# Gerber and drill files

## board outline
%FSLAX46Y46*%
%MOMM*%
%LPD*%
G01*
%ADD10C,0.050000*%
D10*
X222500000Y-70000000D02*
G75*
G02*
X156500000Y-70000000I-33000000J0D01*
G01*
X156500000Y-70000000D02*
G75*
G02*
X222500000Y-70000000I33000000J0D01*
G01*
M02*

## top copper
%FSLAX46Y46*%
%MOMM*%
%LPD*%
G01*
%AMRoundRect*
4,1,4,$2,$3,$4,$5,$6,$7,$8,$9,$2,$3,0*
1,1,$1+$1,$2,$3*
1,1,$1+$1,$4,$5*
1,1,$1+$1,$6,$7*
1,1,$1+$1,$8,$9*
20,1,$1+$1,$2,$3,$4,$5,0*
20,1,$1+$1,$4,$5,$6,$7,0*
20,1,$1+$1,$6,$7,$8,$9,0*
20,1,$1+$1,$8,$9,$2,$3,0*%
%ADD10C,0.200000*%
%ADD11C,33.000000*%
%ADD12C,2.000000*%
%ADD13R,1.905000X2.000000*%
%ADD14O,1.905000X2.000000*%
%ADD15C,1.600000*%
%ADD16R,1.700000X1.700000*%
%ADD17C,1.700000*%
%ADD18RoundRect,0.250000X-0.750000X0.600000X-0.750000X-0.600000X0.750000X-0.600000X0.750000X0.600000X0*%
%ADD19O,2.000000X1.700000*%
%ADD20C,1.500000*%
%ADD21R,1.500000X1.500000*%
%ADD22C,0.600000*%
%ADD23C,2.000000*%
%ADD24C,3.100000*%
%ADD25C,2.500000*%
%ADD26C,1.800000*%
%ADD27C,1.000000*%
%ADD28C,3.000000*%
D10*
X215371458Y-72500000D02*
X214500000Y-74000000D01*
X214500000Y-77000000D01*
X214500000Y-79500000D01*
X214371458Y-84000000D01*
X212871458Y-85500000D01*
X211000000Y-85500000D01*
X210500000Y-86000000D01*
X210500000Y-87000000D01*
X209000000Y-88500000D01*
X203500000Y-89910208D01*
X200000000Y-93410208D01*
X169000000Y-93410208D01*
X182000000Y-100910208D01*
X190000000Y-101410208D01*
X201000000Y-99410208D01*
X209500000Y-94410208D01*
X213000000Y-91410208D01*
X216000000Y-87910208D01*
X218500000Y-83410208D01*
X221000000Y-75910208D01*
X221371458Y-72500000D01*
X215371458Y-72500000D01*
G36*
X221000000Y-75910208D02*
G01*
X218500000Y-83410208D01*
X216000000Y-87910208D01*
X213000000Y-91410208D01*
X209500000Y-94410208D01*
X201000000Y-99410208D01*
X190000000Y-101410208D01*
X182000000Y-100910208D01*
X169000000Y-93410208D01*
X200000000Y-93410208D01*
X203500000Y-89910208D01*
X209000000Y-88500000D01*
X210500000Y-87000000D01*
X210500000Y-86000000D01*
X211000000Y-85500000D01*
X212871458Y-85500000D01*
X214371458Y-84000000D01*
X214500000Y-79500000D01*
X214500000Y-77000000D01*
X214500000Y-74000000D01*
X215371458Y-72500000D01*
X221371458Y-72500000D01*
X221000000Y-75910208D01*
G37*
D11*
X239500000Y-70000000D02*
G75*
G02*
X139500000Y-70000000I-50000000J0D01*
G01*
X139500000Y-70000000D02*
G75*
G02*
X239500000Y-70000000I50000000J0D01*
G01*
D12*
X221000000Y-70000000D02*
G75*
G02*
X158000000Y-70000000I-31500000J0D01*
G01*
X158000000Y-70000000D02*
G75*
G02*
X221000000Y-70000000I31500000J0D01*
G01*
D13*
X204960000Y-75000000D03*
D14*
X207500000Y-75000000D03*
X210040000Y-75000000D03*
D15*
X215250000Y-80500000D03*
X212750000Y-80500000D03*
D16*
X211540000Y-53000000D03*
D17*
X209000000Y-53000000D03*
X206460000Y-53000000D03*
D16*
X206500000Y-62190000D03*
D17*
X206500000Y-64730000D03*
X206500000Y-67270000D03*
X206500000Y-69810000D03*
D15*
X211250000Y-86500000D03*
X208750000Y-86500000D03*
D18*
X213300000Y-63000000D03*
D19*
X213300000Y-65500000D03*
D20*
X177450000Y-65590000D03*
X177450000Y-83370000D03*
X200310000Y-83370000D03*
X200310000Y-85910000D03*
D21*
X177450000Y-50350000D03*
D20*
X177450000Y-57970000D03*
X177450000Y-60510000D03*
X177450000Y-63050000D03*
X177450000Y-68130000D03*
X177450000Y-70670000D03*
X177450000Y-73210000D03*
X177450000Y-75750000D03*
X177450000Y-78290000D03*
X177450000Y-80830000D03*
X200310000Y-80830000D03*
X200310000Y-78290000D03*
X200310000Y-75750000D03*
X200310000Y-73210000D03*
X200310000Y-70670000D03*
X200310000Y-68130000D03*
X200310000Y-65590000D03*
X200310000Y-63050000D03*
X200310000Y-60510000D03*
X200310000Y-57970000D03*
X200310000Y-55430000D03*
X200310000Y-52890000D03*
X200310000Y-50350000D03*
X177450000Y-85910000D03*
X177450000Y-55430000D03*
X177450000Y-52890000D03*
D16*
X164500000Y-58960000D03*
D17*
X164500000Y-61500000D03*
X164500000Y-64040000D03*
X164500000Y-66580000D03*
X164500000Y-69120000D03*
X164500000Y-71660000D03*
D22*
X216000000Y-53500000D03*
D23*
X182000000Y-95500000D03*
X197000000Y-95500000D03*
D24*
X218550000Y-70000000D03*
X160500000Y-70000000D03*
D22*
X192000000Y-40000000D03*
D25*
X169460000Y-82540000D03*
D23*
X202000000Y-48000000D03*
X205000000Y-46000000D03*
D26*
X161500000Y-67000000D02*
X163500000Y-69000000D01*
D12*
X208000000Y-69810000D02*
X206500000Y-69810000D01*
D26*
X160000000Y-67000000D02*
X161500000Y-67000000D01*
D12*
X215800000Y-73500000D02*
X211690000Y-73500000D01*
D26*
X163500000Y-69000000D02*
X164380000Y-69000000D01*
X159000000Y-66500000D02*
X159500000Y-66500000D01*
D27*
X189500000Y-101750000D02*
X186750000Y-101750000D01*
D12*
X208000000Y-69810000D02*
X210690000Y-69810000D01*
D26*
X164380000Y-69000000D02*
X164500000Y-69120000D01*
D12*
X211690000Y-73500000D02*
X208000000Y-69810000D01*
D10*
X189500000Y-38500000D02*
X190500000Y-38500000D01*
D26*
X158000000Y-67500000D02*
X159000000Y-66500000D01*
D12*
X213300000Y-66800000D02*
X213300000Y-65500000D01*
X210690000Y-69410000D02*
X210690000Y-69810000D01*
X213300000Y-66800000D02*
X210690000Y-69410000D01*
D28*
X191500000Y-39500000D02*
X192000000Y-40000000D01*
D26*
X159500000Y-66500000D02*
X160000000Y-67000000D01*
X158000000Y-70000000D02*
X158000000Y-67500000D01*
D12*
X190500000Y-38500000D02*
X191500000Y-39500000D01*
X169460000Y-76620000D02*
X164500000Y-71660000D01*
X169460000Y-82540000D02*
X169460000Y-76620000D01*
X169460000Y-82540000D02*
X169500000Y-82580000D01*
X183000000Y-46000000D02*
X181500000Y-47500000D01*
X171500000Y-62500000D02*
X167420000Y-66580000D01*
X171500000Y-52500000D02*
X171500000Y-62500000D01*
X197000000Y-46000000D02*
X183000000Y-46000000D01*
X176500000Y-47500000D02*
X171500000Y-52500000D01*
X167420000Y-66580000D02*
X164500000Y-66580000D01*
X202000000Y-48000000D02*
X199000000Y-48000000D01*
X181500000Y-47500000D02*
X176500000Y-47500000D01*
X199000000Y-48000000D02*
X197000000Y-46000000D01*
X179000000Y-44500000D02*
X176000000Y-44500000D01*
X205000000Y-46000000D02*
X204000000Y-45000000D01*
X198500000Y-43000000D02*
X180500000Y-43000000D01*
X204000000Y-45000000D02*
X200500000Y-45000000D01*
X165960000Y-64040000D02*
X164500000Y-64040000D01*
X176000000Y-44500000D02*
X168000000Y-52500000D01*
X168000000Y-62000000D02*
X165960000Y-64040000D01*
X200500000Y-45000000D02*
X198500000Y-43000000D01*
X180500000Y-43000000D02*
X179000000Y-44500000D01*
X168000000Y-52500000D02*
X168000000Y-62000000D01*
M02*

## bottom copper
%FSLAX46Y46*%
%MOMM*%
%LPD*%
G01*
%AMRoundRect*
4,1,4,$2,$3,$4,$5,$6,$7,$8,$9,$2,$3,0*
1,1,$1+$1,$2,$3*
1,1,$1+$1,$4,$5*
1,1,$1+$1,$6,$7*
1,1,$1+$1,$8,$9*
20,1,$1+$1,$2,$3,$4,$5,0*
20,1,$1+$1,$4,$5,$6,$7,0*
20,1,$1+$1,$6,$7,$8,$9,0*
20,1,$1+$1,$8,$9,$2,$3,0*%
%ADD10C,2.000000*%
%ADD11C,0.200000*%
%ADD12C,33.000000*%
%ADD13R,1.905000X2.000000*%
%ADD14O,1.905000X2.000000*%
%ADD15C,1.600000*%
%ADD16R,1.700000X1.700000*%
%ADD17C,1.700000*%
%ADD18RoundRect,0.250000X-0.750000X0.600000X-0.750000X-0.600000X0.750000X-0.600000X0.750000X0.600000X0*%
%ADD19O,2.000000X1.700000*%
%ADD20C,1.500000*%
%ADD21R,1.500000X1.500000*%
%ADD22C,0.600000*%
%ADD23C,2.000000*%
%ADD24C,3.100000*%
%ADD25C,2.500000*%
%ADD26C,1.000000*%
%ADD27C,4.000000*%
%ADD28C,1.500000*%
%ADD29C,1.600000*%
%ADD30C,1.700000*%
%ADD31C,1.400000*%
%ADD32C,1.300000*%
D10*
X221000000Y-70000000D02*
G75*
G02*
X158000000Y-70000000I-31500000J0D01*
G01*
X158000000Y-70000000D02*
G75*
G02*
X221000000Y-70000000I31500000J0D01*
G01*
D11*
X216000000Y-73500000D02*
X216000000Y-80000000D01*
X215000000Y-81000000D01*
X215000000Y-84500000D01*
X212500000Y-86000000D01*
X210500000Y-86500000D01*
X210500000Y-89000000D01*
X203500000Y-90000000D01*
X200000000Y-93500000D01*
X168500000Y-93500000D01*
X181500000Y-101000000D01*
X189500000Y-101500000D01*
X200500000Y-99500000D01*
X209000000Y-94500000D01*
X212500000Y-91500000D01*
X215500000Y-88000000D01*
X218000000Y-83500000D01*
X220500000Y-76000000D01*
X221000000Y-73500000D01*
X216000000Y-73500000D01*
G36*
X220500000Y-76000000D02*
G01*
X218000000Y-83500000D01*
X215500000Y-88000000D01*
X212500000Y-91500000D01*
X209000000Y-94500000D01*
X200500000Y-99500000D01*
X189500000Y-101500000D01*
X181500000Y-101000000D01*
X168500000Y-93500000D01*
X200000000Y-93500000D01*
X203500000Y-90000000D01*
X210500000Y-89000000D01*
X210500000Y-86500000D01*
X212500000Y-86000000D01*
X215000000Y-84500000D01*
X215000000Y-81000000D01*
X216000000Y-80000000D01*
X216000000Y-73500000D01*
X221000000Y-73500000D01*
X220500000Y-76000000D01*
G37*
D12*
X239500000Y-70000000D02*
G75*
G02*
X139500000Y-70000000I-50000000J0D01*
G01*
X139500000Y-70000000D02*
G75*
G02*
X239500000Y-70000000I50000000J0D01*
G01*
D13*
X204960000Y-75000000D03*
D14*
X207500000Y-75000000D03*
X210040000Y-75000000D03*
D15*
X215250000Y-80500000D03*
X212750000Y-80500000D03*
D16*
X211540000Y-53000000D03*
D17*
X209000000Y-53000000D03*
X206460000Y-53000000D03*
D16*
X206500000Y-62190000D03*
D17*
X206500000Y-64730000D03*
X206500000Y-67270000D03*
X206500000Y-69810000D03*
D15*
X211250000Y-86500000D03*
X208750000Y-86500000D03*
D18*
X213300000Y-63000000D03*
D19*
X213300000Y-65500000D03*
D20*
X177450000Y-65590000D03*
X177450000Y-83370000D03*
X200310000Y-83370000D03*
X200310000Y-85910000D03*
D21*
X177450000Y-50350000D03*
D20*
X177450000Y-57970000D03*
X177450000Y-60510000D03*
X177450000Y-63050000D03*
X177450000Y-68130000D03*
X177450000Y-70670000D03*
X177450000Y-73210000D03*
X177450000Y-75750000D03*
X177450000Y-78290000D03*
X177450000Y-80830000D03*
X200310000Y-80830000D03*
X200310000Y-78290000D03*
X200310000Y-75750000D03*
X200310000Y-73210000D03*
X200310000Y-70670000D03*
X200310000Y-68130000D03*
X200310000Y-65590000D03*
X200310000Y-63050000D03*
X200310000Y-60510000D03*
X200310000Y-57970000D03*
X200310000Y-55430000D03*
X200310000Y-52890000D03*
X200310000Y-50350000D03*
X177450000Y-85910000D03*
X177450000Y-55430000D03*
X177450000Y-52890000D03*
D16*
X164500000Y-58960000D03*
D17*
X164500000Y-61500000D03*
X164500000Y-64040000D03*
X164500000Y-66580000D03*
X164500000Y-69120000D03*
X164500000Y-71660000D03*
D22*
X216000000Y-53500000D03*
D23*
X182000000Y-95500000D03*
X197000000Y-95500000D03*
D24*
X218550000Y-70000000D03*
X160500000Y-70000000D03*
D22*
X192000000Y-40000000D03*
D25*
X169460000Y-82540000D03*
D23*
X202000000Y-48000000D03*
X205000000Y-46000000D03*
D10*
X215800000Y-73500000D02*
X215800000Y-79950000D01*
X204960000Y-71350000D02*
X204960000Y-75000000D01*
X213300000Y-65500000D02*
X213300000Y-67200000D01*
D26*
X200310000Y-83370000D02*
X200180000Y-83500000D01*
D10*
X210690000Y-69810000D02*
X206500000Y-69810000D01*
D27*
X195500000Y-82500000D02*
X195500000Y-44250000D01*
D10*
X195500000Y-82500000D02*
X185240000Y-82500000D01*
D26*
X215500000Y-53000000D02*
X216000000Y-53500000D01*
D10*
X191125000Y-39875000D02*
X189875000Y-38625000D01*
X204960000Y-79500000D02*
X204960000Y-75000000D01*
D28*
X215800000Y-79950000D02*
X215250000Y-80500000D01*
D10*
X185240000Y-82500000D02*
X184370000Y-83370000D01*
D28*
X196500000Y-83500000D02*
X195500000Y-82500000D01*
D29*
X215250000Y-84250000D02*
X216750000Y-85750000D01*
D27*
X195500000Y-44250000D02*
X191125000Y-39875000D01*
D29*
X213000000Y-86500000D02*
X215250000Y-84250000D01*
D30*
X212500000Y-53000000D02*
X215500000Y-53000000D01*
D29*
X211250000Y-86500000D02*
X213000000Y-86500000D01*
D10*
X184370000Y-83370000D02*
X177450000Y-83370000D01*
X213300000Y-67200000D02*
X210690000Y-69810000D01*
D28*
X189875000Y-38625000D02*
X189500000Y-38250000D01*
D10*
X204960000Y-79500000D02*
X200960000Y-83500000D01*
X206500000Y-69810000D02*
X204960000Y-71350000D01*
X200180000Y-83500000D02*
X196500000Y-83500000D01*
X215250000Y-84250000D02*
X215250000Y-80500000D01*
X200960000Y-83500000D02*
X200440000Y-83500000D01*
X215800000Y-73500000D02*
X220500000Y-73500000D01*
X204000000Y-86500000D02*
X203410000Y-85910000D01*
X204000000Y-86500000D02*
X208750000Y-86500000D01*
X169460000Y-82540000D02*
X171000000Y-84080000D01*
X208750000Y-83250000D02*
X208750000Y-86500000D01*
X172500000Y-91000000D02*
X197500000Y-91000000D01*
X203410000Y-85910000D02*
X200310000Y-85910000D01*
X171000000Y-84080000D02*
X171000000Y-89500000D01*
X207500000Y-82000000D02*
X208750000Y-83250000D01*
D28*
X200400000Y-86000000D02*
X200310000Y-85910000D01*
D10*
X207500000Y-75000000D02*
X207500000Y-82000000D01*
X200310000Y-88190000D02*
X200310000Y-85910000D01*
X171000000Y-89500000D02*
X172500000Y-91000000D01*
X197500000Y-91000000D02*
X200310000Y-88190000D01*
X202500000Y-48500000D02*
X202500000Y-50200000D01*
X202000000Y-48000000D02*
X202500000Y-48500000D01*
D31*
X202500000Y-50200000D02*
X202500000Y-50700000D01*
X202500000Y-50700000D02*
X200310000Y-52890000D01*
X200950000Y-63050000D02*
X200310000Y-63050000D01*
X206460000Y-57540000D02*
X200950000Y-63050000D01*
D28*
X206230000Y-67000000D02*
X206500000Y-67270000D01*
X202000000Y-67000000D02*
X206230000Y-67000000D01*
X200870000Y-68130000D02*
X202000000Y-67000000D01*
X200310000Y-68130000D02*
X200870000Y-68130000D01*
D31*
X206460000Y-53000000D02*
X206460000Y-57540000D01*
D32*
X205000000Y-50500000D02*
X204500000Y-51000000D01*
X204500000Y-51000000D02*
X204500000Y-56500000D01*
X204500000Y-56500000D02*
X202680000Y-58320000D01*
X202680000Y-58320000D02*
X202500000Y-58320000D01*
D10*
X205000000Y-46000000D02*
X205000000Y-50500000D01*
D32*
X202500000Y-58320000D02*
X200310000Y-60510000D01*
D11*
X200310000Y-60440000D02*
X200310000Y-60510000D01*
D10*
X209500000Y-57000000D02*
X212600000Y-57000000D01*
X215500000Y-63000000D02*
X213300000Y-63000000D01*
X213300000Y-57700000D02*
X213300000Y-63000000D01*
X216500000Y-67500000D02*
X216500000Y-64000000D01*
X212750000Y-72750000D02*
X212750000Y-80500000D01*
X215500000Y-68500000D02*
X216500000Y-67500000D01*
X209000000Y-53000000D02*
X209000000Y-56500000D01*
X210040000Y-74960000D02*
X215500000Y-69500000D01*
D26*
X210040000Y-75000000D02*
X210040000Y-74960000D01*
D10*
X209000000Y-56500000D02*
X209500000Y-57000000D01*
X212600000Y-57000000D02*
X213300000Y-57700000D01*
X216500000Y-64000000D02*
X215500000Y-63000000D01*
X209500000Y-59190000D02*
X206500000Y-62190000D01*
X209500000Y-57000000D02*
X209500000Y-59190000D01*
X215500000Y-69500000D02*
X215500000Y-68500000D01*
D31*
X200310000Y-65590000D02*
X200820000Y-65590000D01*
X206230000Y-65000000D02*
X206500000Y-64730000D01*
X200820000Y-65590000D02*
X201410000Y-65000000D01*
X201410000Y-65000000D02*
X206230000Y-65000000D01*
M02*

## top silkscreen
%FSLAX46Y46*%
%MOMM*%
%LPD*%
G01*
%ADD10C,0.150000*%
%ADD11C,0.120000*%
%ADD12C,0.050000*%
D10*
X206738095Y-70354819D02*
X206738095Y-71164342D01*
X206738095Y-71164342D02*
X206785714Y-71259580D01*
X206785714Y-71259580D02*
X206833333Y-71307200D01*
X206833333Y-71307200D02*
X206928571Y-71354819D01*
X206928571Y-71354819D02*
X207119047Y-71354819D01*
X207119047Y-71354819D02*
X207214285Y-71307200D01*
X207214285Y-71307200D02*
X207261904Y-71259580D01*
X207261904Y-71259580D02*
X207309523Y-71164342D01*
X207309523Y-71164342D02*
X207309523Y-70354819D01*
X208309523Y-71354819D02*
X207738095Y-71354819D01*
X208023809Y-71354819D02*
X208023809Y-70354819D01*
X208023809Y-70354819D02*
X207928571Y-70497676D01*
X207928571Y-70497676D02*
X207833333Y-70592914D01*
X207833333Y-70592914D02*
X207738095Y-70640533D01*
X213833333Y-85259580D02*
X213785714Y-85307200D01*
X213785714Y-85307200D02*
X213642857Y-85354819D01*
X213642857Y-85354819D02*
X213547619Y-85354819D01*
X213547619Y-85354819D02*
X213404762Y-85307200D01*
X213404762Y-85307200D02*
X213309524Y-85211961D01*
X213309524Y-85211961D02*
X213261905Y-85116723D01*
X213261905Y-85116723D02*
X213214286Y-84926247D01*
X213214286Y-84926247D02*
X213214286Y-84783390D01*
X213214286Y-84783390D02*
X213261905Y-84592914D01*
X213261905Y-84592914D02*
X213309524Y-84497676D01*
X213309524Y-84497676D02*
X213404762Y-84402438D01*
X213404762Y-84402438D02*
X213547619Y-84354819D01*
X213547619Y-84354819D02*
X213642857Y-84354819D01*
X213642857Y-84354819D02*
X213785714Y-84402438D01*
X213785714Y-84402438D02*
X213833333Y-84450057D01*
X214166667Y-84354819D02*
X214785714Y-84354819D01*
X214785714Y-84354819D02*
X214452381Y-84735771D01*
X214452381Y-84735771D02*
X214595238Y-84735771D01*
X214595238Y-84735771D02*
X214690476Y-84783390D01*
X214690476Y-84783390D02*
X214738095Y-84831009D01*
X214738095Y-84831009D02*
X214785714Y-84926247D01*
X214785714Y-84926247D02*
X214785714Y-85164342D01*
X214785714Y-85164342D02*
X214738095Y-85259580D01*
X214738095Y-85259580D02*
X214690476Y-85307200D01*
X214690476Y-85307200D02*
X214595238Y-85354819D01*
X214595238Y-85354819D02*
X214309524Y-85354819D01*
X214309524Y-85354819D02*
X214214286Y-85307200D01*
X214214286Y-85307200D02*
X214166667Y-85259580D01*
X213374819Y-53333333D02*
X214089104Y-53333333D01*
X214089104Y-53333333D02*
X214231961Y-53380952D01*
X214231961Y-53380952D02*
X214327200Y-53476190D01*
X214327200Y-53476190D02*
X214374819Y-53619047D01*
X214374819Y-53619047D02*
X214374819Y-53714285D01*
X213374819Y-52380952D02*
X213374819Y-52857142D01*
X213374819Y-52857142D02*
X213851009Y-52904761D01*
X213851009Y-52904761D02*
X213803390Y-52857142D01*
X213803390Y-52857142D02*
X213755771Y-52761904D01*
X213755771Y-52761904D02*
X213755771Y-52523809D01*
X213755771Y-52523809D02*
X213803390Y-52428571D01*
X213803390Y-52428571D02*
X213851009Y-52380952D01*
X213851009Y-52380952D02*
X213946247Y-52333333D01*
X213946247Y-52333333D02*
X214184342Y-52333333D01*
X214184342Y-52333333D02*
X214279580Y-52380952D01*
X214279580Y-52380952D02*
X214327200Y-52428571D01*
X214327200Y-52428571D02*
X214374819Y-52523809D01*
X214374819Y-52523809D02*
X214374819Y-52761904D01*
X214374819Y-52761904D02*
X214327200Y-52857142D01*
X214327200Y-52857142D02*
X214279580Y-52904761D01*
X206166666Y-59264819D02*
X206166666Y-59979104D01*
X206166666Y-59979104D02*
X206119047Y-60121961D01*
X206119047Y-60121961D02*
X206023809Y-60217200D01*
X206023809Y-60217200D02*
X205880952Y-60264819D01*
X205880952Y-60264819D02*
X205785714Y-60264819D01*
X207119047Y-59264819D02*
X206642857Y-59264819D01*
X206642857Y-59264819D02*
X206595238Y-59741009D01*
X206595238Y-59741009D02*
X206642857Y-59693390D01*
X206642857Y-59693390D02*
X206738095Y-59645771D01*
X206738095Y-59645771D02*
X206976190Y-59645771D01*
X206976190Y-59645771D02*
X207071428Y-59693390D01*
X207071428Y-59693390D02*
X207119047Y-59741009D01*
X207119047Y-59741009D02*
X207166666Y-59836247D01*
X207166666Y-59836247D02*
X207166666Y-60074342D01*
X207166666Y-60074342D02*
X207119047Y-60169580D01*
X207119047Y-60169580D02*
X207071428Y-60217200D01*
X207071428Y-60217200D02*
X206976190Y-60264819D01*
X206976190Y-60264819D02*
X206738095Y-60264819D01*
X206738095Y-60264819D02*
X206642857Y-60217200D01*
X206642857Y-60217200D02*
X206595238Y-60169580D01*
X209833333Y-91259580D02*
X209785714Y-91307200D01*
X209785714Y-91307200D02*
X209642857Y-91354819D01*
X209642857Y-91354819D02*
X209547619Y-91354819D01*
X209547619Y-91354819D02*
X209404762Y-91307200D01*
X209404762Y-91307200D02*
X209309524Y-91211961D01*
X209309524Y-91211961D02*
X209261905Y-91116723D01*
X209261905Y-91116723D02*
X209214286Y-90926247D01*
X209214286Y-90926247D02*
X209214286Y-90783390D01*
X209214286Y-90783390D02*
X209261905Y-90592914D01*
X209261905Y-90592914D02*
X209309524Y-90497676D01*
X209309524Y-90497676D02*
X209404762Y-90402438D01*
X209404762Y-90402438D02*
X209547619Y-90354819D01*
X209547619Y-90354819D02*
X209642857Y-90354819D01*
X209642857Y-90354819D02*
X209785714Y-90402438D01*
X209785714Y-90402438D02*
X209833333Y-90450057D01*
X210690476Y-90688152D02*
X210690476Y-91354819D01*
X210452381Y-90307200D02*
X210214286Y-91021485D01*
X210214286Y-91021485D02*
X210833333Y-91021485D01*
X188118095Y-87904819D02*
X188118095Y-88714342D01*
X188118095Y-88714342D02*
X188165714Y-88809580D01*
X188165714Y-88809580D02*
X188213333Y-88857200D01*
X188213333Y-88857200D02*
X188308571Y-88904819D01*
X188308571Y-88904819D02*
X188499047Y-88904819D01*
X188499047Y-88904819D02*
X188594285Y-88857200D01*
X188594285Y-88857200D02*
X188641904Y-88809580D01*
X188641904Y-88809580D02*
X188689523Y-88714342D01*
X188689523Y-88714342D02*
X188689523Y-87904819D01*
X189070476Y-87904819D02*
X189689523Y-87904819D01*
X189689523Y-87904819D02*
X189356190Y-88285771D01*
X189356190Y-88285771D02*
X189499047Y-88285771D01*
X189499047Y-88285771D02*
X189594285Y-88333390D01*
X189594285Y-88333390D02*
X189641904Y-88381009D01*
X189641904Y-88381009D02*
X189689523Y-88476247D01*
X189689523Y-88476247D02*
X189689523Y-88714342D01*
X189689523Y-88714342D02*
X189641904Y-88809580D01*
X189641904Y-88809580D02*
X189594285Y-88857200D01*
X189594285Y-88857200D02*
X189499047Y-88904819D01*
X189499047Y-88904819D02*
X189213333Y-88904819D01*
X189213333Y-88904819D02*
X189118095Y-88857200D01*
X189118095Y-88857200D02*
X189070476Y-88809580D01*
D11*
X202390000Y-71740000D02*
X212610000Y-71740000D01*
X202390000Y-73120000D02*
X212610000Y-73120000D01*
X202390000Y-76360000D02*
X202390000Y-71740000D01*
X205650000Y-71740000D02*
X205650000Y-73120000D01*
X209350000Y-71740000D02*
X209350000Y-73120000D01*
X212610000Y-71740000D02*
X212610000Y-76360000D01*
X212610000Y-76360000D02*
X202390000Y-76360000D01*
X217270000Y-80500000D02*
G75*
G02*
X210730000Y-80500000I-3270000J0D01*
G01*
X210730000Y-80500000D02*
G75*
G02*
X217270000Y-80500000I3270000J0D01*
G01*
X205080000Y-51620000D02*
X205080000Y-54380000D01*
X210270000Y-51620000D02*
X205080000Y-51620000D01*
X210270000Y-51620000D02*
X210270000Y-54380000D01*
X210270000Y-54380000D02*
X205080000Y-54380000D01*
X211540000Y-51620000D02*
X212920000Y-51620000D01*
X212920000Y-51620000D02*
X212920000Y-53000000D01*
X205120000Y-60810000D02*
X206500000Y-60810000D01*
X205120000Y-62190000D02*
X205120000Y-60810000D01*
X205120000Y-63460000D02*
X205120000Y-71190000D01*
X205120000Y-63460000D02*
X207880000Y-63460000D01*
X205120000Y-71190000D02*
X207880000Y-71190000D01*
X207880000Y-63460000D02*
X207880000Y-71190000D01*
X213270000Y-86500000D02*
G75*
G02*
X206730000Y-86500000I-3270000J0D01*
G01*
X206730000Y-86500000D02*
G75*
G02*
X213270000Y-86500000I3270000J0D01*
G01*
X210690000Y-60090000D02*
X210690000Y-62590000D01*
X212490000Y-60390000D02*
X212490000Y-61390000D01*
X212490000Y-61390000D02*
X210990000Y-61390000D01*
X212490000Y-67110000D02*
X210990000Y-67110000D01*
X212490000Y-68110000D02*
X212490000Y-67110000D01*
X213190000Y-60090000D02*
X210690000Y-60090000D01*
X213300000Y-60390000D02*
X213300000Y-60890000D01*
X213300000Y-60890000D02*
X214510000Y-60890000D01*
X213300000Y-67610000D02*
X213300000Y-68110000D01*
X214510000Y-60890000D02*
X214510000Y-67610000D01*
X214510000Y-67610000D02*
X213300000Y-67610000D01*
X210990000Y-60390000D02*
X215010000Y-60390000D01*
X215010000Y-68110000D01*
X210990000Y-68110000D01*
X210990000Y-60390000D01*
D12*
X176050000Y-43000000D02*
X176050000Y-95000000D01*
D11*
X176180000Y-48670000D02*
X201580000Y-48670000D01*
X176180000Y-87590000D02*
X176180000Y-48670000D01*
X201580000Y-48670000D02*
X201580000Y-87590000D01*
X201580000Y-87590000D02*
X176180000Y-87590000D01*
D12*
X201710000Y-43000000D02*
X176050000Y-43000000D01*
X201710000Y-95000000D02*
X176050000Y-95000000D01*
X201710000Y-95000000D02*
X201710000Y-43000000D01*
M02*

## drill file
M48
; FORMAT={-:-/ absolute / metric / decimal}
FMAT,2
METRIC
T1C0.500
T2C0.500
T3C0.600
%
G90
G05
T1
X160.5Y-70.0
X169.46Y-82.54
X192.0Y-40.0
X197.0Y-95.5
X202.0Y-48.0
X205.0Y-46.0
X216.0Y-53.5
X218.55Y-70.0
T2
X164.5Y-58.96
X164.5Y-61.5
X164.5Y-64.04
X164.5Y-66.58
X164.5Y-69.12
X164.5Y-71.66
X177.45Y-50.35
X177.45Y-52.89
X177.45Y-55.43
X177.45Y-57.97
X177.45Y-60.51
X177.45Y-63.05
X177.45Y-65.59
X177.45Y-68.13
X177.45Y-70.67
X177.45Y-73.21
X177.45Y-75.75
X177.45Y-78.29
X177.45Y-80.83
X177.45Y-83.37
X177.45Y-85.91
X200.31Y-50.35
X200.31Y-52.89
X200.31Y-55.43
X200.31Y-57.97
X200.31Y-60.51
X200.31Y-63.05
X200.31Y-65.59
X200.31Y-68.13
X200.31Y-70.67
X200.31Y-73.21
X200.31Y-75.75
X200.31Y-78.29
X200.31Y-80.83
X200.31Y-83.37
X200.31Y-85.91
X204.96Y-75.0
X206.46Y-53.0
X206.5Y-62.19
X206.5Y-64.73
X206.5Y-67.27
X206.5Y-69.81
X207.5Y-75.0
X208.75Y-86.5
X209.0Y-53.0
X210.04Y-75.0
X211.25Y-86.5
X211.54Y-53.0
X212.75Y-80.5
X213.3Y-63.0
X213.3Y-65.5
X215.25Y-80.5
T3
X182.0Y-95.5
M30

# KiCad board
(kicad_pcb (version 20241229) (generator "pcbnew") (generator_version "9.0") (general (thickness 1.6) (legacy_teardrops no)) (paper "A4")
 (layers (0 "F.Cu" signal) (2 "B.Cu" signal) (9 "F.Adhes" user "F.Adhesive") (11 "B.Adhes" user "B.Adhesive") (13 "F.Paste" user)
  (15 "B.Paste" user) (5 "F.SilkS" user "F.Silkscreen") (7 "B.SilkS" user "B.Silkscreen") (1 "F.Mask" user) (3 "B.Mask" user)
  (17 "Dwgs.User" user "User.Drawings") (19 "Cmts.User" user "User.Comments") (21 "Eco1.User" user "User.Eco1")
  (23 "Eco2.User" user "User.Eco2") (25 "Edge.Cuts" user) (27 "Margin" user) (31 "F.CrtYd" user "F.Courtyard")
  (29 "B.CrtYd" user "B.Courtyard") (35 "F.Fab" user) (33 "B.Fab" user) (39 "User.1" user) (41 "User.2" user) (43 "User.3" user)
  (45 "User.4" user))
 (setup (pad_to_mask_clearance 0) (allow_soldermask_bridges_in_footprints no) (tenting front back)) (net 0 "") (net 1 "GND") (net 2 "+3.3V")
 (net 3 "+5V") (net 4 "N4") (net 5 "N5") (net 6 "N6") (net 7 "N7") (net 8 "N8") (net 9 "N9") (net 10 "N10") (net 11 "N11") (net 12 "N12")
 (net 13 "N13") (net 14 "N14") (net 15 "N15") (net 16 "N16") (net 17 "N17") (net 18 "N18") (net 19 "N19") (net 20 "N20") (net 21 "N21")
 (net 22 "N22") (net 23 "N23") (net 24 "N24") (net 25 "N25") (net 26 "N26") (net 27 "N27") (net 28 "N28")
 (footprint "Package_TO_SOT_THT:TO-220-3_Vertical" (layer "F.Cu") (at 204.96 75)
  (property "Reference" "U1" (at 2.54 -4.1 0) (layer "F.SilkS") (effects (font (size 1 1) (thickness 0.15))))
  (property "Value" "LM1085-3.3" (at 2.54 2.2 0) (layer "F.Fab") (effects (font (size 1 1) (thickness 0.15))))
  (fp_line (start -2.57 -3.26) (end 7.65 -3.26) (stroke (width 0.12) (type solid)) (layer "F.SilkS"))
  (fp_line (start -2.57 -1.88) (end 7.65 -1.88) (stroke (width 0.12) (type solid)) (layer "F.SilkS"))
  (fp_line (start -2.57 1.36) (end -2.57 -3.26) (stroke (width 0.12) (type solid)) (layer "F.SilkS"))
  (fp_line (start 0.69 -3.26) (end 0.69 -1.88) (stroke (width 0.12) (type solid)) (layer "F.SilkS"))
  (fp_line (start 4.39 -3.26) (end 4.39 -1.88) (stroke (width 0.12) (type solid)) (layer "F.SilkS"))
  (fp_line (start 7.65 -3.26) (end 7.65 1.36) (stroke (width 0.12) (type solid)) (layer "F.SilkS"))
  (fp_line (start 7.65 1.36) (end -2.57 1.36) (stroke (width 0.12) (type solid)) (layer "F.SilkS"))
  (pad "1" thru_hole rect (at 0 0) (size 1.905 2) (drill 0.5) (layers "*.Cu" "*.Mask") (remove_unused_layers no) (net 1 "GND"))
  (pad "2" thru_hole oval (at 2.54 0) (size 1.905 2) (drill 0.5) (layers "*.Cu" "*.Mask") (remove_unused_layers no) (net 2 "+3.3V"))
  (pad "3" thru_hole oval (at 5.08 0) (size 1.905 2) (drill 0.5) (layers "*.Cu" "*.Mask") (remove_unused_layers no) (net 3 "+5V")))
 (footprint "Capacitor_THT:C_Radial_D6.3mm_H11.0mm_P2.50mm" (layer "F.Cu") (at 215.25 80.5 180)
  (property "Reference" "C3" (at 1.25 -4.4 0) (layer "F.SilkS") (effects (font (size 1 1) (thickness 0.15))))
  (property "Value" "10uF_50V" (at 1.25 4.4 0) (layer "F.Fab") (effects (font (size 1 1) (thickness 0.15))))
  (fp_circle (center 1.25 0) (end 4.52 0) (stroke (width 0.12) (type solid)) (fill no) (layer "F.SilkS"))
  (pad "1" thru_hole circle (at 0 0 180) (size 1.6 1.6) (drill 0.5) (layers "*.Cu" "*.Mask") (remove_unused_layers no) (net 1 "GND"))
  (pad "2" thru_hole circle (at 2.5 0 180) (size 1.6 1.6) (drill 0.5) (layers "*.Cu" "*.Mask") (remove_unused_layers no) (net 3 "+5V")))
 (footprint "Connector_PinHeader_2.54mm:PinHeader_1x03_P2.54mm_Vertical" (layer "F.Cu") (at 211.54 53 -90)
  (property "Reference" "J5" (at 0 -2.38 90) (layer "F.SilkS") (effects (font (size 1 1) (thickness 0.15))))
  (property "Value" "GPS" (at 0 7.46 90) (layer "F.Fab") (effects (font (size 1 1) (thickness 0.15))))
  (fp_line (start -1.38 6.46) (end 1.38 6.46) (stroke (width 0.12) (type solid)) (layer "F.SilkS"))
  (fp_line (start -1.38 1.27) (end -1.38 6.46) (stroke (width 0.12) (type solid)) (layer "F.SilkS"))
  (fp_line (start -1.38 1.27) (end 1.38 1.27) (stroke (width 0.12) (type solid)) (layer "F.SilkS"))
  (fp_line (start 1.38 1.27) (end 1.38 6.46) (stroke (width 0.12) (type solid)) (layer "F.SilkS"))
  (fp_line (start -1.38 0) (end -1.38 -1.38) (stroke (width 0.12) (type solid)) (layer "F.SilkS"))
  (fp_line (start -1.38 -1.38) (end 0 -1.38) (stroke (width 0.12) (type solid)) (layer "F.SilkS"))
  (pad "1" thru_hole rect (at 0 0 270) (size 1.7 1.7) (drill 0.5) (layers "*.Cu" "*.Mask") (remove_unused_layers no) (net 1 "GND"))
  (pad "2" thru_hole circle (at 0 2.54 270) (size 1.7 1.7) (drill 0.5) (layers "*.Cu" "*.Mask") (remove_unused_layers no) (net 3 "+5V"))
  (pad "3" thru_hole circle (at 0 5.08 270) (size 1.7 1.7) (drill 0.5) (layers "*.Cu" "*.Mask") (remove_unused_layers no) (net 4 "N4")))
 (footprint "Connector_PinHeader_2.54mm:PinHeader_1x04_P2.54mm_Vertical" (layer "F.Cu") (at 206.5 62.19)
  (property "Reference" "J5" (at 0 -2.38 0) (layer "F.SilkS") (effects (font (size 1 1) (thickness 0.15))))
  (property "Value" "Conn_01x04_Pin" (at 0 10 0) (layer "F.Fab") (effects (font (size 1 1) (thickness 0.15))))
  (fp_line (start -1.38 -1.38) (end 0 -1.38) (stroke (width 0.12) (type solid)) (layer "F.SilkS"))
  (fp_line (start -1.38 0) (end -1.38 -1.38) (stroke (width 0.12) (type solid)) (layer "F.SilkS"))
  (fp_line (start -1.38 1.27) (end -1.38 9) (stroke (width 0.12) (type solid)) (layer "F.SilkS"))
  (fp_line (start -1.38 1.27) (end 1.38 1.27) (stroke (width 0.12) (type solid)) (layer "F.SilkS"))
  (fp_line (start -1.38 9) (end 1.38 9) (stroke (width 0.12) (type solid)) (layer "F.SilkS"))
  (fp_line (start 1.38 1.27) (end 1.38 9) (stroke (width 0.12) (type solid)) (layer "F.SilkS"))
  (pad "1" thru_hole rect (at 0 0) (size 1.7 1.7) (drill 0.5) (layers "*.Cu" "*.Mask") (remove_unused_layers no) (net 3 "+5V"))
  (pad "2" thru_hole circle (at 0 2.54) (size 1.7 1.7) (drill 0.5) (layers "*.Cu" "*.Mask") (remove_unused_layers no) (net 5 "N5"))
  (pad "3" thru_hole circle (at 0 5.08) (size 1.7 1.7) (drill 0.5) (layers "*.Cu" "*.Mask") (remove_unused_layers no) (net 4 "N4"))
  (pad "4" thru_hole circle (at 0 7.62) (size 1.7 1.7) (drill 0.5) (layers "*.Cu" "*.Mask") (remove_unused_layers no) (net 1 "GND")))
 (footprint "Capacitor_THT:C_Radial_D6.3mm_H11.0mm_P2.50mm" (layer "F.Cu") (at 211.25 86.5 180)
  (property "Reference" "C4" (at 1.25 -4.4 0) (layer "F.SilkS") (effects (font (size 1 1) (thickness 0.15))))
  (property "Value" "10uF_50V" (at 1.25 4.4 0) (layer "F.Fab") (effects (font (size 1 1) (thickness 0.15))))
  (fp_circle (center 1.25 0) (end 4.52 0) (stroke (width 0.12) (type solid)) (fill no) (layer "F.SilkS"))
  (pad "1" thru_hole circle (at 0 0 180) (size 1.6 1.6) (drill 0.5) (layers "*.Cu" "*.Mask") (remove_unused_layers no) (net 1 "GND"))
  (pad "2" thru_hole circle (at 2.5 0 180) (size 1.6 1.6) (drill 0.5) (layers "*.Cu" "*.Mask") (remove_unused_layers no) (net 2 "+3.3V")))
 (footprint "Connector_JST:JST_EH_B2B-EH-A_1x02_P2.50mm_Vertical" (layer "F.Cu") (at 213.3 63 -90)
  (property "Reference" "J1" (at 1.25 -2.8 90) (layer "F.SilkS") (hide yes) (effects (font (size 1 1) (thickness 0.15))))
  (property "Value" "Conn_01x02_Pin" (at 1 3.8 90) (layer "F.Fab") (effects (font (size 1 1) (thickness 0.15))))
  (fp_line (start -2.91 2.61) (end -0.41 2.61) (stroke (width 0.12) (type solid)) (layer "F.SilkS"))
  (fp_line (start -2.61 0.81) (end -1.61 0.81) (stroke (width 0.12) (type solid)) (layer "F.SilkS"))
  (fp_line (start -1.61 0.81) (end -1.61 2.31) (stroke (width 0.12) (type solid)) (layer "F.SilkS"))
  (fp_line (start 4.11 0.81) (end 4.11 2.31) (stroke (width 0.12) (type solid)) (layer "F.SilkS"))
  (fp_line (start 5.11 0.81) (end 4.11 0.81) (stroke (width 0.12) (type solid)) (layer "F.SilkS"))
  (fp_line (start -2.91 0.11) (end -2.91 2.61) (stroke (width 0.12) (type solid)) (layer "F.SilkS"))
  (fp_line (start -2.61 0) (end -2.11 0) (stroke (width 0.12) (type solid)) (layer "F.SilkS"))
  (fp_line (start -2.11 0) (end -2.11 -1.21) (stroke (width 0.12) (type solid)) (layer "F.SilkS"))
  (fp_line (start 4.61 0) (end 5.11 0) (stroke (width 0.12) (type solid)) (layer "F.SilkS"))
  (fp_line (start -2.11 -1.21) (end 4.61 -1.21) (stroke (width 0.12) (type solid)) (layer "F.SilkS"))
  (fp_line (start 4.61 -1.21) (end 4.61 0) (stroke (width 0.12) (type solid)) (layer "F.SilkS"))
  (fp_rect (start -2.61 -1.71) (end 5.11 2.31) (stroke (width 0.12) (type solid)) (fill no) (layer "F.SilkS"))
  (pad "1" thru_hole roundrect (at 0 0 270) (size 1.7 2) (drill 0.5) (layers "*.Cu" "*.Mask") (remove_unused_layers no)
   (roundrect_rratio 0.147059) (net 3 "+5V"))
  (pad "2" thru_hole oval (at 2.5 0 270) (size 1.7 2) (drill 0.5) (layers "*.Cu" "*.Mask") (remove_unused_layers no) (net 1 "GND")))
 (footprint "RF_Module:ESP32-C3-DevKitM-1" (layer "F.Cu") (at 177.45 50.35)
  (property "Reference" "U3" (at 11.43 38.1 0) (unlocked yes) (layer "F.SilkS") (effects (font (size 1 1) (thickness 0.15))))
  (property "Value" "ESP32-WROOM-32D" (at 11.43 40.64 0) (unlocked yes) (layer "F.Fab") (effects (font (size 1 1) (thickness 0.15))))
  (fp_line (start -1.4 -7.35) (end -1.4 44.65) (stroke (width 0.05) (type solid)) (layer "F.SilkS"))
  (fp_line (start -1.27 -1.68) (end 24.13 -1.68) (stroke (width 0.12) (type solid)) (layer "F.SilkS"))
  (fp_line (start -1.27 37.24) (end -1.27 -1.68) (stroke (width 0.12) (type solid)) (layer "F.SilkS"))
  (fp_line (start 24.13 -1.68) (end 24.13 37.24) (stroke (width 0.12) (type solid)) (layer "F.SilkS"))
  (fp_line (start 24.13 37.24) (end -1.27 37.24) (stroke (width 0.12) (type solid)) (layer "F.SilkS"))
  (fp_line (start 24.26 -7.35) (end -1.4 -7.35) (stroke (width 0.05) (type solid)) (layer "F.SilkS"))
  (fp_line (start 24.26 44.65) (end -1.4 44.65) (stroke (width 0.05) (type solid)) (layer "F.SilkS"))
  (fp_line (start 24.26 44.65) (end 24.26 -7.35) (stroke (width 0.05) (type solid)) (layer "F.SilkS"))
  (pad "" thru_hole circle (at 0 15.24) (size 1.5 1.5) (drill 0.5) (layers "*.Cu" "*.Mask") (remove_unused_layers no))
  (pad "1" thru_hole circle (at 0 33.02) (size 1.5 1.5) (drill 0.5) (layers "*.Cu" "*.Mask") (remove_unused_layers no) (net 1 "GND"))
  (pad "1" thru_hole circle (at 22.86 33.02) (size 1.5 1.5) (drill 0.5) (layers "*.Cu" "*.Mask") (remove_unused_layers no) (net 1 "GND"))
  (pad "2" thru_hole circle (at 22.86 35.56) (size 1.5 1.5) (drill 0.5) (layers "*.Cu" "*.Mask") (remove_unused_layers no) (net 2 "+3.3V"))
  (pad "3" thru_hole rect (at 0 0) (size 1.5 1.5) (drill 0.5) (layers "*.Cu" "*.Mask") (remove_unused_layers no) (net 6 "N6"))
  (pad "6" thru_hole circle (at 0 7.62) (size 1.5 1.5) (drill 0.5) (layers "*.Cu" "*.Mask") (remove_unused_layers no) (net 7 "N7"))
  (pad "7" thru_hole circle (at 0 10.16) (size 1.5 1.5) (drill 0.5) (layers "*.Cu" "*.Mask") (remove_unused_layers no) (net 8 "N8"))
  (pad "8" thru_hole circle (at 0 12.7) (size 1.5 1.5) (drill 0.5) (layers "*.Cu" "*.Mask") (remove_unused_layers no) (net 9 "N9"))
  (pad "10" thru_hole circle (at 0 17.78) (size 1.5 1.5) (drill 0.5) (layers "*.Cu" "*.Mask") (remove_unused_layers no) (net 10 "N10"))
  (pad "11" thru_hole circle (at 0 20.32) (size 1.5 1.5) (drill 0.5) (layers "*.Cu" "*.Mask") (remove_unused_layers no) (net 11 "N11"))
  (pad "12" thru_hole circle (at 0 22.86) (size 1.5 1.5) (drill 0.5) (layers "*.Cu" "*.Mask") (remove_unused_layers no) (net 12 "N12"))
  (pad "13" thru_hole circle (at 0 25.4) (size 1.5 1.5) (drill 0.5) (layers "*.Cu" "*.Mask") (remove_unused_layers no) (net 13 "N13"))
  (pad "14" thru_hole circle (at 0 27.94) (size 1.5 1.5) (drill 0.5) (layers "*.Cu" "*.Mask") (remove_unused_layers no) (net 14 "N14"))
  (pad "16" thru_hole circle (at 0 30.48) (size 1.5 1.5) (drill 0.5) (layers "*.Cu" "*.Mask") (remove_unused_layers no) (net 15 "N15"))
  (pad "23" thru_hole circle (at 22.86 30.48) (size 1.5 1.5) (drill 0.5) (layers "*.Cu" "*.Mask") (remove_unused_layers no) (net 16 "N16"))
  (pad "24" thru_hole circle (at 22.86 27.94) (size 1.5 1.5) (drill 0.5) (layers "*.Cu" "*.Mask") (remove_unused_layers no) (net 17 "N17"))
  (pad "26" thru_hole circle (at 22.86 25.4) (size 1.5 1.5) (drill 0.5) (layers "*.Cu" "*.Mask") (remove_unused_layers no) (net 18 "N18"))
  (pad "27" thru_hole circle (at 22.86 22.86) (size 1.5 1.5) (drill 0.5) (layers "*.Cu" "*.Mask") (remove_unused_layers no) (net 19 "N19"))
  (pad "28" thru_hole circle (at 22.86 20.32) (size 1.5 1.5) (drill 0.5) (layers "*.Cu" "*.Mask") (remove_unused_layers no) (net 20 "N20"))
  (pad "29" thru_hole circle (at 22.86 17.78) (size 1.5 1.5) (drill 0.5) (layers "*.Cu" "*.Mask") (remove_unused_layers no) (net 4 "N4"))
  (pad "30" thru_hole circle (at 22.86 15.24) (size 1.5 1.5) (drill 0.5) (layers "*.Cu" "*.Mask") (remove_unused_layers no) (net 5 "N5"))
  (pad "31" thru_hole circle (at 22.86 12.7) (size 1.5 1.5) (drill 0.5) (layers "*.Cu" "*.Mask") (remove_unused_layers no) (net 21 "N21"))
  (pad "33" thru_hole circle (at 22.86 10.16) (size 1.5 1.5) (drill 0.5) (layers "*.Cu" "*.Mask") (remove_unused_layers no) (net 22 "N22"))
  (pad "34" thru_hole circle (at 22.86 7.62) (size 1.5 1.5) (drill 0.5) (layers "*.Cu" "*.Mask") (remove_unused_layers no) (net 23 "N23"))
  (pad "35" thru_hole circle (at 22.86 5.08) (size 1.5 1.5) (drill 0.5) (layers "*.Cu" "*.Mask") (remove_unused_layers no) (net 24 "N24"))
  (pad "36" thru_hole circle (at 22.86 2.54) (size 1.5 1.5) (drill 0.5) (layers "*.Cu" "*.Mask") (remove_unused_layers no) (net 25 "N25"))
  (pad "37" thru_hole circle (at 22.86 0) (size 1.5 1.5) (drill 0.5) (layers "*.Cu" "*.Mask") (remove_unused_layers no) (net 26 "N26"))
  (pad "50" thru_hole circle (at 0 35.56) (size 1.5 1.5) (drill 0.5) (layers "*.Cu" "*.Mask") (remove_unused_layers no))
  (pad "52" thru_hole circle (at 0 5.08) (size 1.5 1.5) (drill 0.5) (layers "*.Cu" "*.Mask") (remove_unused_layers no))
  (pad "53" thru_hole circle (at 0 2.54) (size 1.5 1.5) (drill 0.5) (layers "*.Cu" "*.Mask") (remove_unused_layers no)))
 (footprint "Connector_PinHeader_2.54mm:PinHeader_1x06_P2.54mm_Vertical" (layer "B.Cu") (at 164.5 58.96 180)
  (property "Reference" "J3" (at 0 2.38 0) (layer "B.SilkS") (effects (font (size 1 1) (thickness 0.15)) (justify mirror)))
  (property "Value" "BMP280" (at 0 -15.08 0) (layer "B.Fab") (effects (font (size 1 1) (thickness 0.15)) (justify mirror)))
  (pad "1" thru_hole rect (at 0 0 180) (size 1.7 1.7) (drill 0.5) (layers "*.Cu" "*.Mask") (remove_unused_layers no) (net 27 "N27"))
  (pad "2" thru_hole circle (at 0 -2.54 180) (size 1.7 1.7) (drill 0.5) (layers "*.Cu" "*.Mask") (remove_unused_layers no) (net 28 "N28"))
  (pad "3" thru_hole circle (at 0 -5.08 180) (size 1.7 1.7) (drill 0.5) (layers "*.Cu" "*.Mask") (remove_unused_layers no) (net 22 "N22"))
  (pad "4" thru_hole circle (at 0 -7.62 180) (size 1.7 1.7) (drill 0.5) (layers "*.Cu" "*.Mask") (remove_unused_layers no) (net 25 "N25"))
  (pad "5" thru_hole circle (at 0 -10.16 180) (size 1.7 1.7) (drill 0.5) (layers "*.Cu" "*.Mask") (remove_unused_layers no) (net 1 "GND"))
  (pad "6" thru_hole circle (at 0 -12.7 180) (size 1.7 1.7) (drill 0.5) (layers "*.Cu" "*.Mask") (remove_unused_layers no) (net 2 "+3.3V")))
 (gr_poly
  (pts (xy 215.371458 72.5) (xy 214.5 74) (xy 214.5 77) (xy 214.5 79.5) (xy 214.371458 84) (xy 212.871458 85.5) (xy 211 85.5) (xy 210.5 86)
   (xy 210.5 87) (xy 209 88.5) (xy 203.5 89.910208) (xy 200 93.410208) (xy 169 93.410208) (xy 182 100.910208) (xy 190 101.410208)
   (xy 201 99.410208) (xy 209.5 94.410208) (xy 213 91.410208) (xy 216 87.910208) (xy 218.5 83.410208) (xy 221 75.910208)
   (xy 221.371458 72.5))
  (stroke (width 0.2) (type solid)) (fill yes) (layer "F.Cu") (net 1))
 (gr_circle (center 189.5 70) (end 239.5 70) (stroke (width 33) (type solid)) (fill no) (layer "F.Cu") (net 1))
 (gr_circle (center 189.5 70) (end 221 70) (stroke (width 2) (type solid)) (fill no) (layer "F.Cu") (net 1))
 (gr_circle (center 189.5 70) (end 221 70) (stroke (width 2) (type solid)) (fill no) (layer "B.Cu") (net 1))
 (gr_poly
  (pts (xy 216 73.5) (xy 216 80) (xy 215 81) (xy 215 84.5) (xy 212.5 86) (xy 210.5 86.5) (xy 210.5 89) (xy 203.5 90) (xy 200 93.5)
   (xy 168.5 93.5) (xy 181.5 101) (xy 189.5 101.5) (xy 200.5 99.5) (xy 209 94.5) (xy 212.5 91.5) (xy 215.5 88) (xy 218 83.5) (xy 220.5 76)
   (xy 221 73.5))
  (stroke (width 0.2) (type solid)) (fill yes) (layer "B.Cu") (net 1))
 (gr_circle (center 189.5 70) (end 239.5 70) (stroke (width 33) (type solid)) (fill no) (layer "B.Cu"))
 (gr_circle (center 189.5 70) (end 222.5 70) (stroke (width 0.05) (type solid)) (fill no) (layer "Edge.Cuts"))
 (segment (start 161.5 67) (end 163.5 69) (width 1.8) (layer "F.Cu") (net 1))
 (segment (start 208 69.81) (end 206.5 69.81) (width 2) (layer "F.Cu") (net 1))
 (segment (start 160 67) (end 161.5 67) (width 1.8) (layer "F.Cu") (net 1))
 (segment (start 215.8 73.5) (end 211.69 73.5) (width 2) (layer "F.Cu") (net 1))
 (segment (start 163.5 69) (end 164.38 69) (width 1.8) (layer "F.Cu") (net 1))
 (segment (start 159 66.5) (end 159.5 66.5) (width 1.8) (layer "F.Cu") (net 1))
 (segment (start 189.5 101.75) (end 186.75 101.75) (width 1) (layer "F.Cu") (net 1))
 (segment (start 208 69.81) (end 210.69 69.81) (width 2) (layer "F.Cu") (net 1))
 (segment (start 164.38 69) (end 164.5 69.12) (width 1.8) (layer "F.Cu") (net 1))
 (segment (start 211.69 73.5) (end 208 69.81) (width 2) (layer "F.Cu") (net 1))
 (segment (start 189.5 38.5) (end 190.5 38.5) (width 0.2) (layer "F.Cu") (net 1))
 (segment (start 158 67.5) (end 159 66.5) (width 1.8) (layer "F.Cu") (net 1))
 (segment (start 213.3 66.8) (end 213.3 65.5) (width 2) (layer "F.Cu") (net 1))
 (segment (start 210.69 69.41) (end 210.69 69.81) (width 2) (layer "F.Cu") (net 1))
 (segment (start 213.3 66.8) (end 210.69 69.41) (width 2) (layer "F.Cu") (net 1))
 (segment (start 191.5 39.5) (end 192 40) (width 3) (layer "F.Cu") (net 1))
 (segment (start 159.5 66.5) (end 160 67) (width 1.8) (layer "F.Cu") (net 1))
 (segment (start 158 70) (end 158 67.5) (width 1.8) (layer "F.Cu") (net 1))
 (segment (start 190.5 38.5) (end 191.5 39.5) (width 2) (layer "F.Cu") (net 1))
 (via (at 216 53.5) (size 0.6) (drill 0.5) (layers "F.Cu" "B.Cu") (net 1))
 (via (at 182 95.5) (size 2) (drill 0.6) (layers "F.Cu" "B.Cu") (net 1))
 (via (at 197 95.5) (size 2) (drill 0.5) (layers "F.Cu" "B.Cu") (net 1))
 (via (at 218.55 70) (size 3.1) (drill 0.5) (layers "F.Cu" "B.Cu") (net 1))
 (via (at 160.5 70) (size 3.1) (drill 0.5) (layers "F.Cu" "B.Cu") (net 1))
 (via (at 192 40) (size 0.6) (drill 0.5) (layers "F.Cu" "B.Cu") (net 1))
 (segment (start 215.8 73.5) (end 215.8 79.95) (width 2) (layer "B.Cu") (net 1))
 (segment (start 204.96 71.35) (end 204.96 75) (width 2) (layer "B.Cu") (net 1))
 (segment (start 213.3 65.5) (end 213.3 67.2) (width 2) (layer "B.Cu") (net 1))
 (segment (start 200.31 83.37) (end 200.18 83.5) (width 1) (layer "B.Cu") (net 1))
 (segment (start 210.69 69.81) (end 206.5 69.81) (width 2) (layer "B.Cu") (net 1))
 (segment (start 195.5 82.5) (end 195.5 44.25) (width 4) (layer "B.Cu") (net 1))
 (segment (start 195.5 82.5) (end 185.24 82.5) (width 2) (layer "B.Cu") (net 1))
 (segment (start 215.5 53) (end 216 53.5) (width 1) (layer "B.Cu") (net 1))
 (segment (start 191.125 39.875) (end 189.875 38.625) (width 2) (layer "B.Cu") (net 1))
 (segment (start 204.96 79.5) (end 204.96 75) (width 2) (layer "B.Cu") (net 1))
 (segment (start 215.8 79.95) (end 215.25 80.5) (width 1.5) (layer "B.Cu") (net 1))
 (segment (start 185.24 82.5) (end 184.37 83.37) (width 2) (layer "B.Cu") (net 1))
 (segment (start 196.5 83.5) (end 195.5 82.5) (width 1.5) (layer "B.Cu") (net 1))
 (segment (start 215.25 84.25) (end 216.75 85.75) (width 1.6) (layer "B.Cu") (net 1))
 (segment (start 195.5 44.25) (end 191.125 39.875) (width 4) (layer "B.Cu") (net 1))
 (segment (start 213 86.5) (end 215.25 84.25) (width 1.6) (layer "B.Cu") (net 1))
 (segment (start 212.5 53) (end 215.5 53) (width 1.7) (layer "B.Cu") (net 1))
 (segment (start 211.25 86.5) (end 213 86.5) (width 1.6) (layer "B.Cu") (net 1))
 (segment (start 184.37 83.37) (end 177.45 83.37) (width 2) (layer "B.Cu") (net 1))
 (segment (start 213.3 67.2) (end 210.69 69.81) (width 2) (layer "B.Cu") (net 1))
 (segment (start 189.875 38.625) (end 189.5 38.25) (width 1.5) (layer "B.Cu") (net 1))
 (segment (start 204.96 79.5) (end 200.96 83.5) (width 2) (layer "B.Cu") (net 1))
 (segment (start 206.5 69.81) (end 204.96 71.35) (width 2) (layer "B.Cu") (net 1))
 (segment (start 200.18 83.5) (end 196.5 83.5) (width 2) (layer "B.Cu") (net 1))
 (segment (start 215.25 84.25) (end 215.25 80.5) (width 2) (layer "B.Cu") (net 1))
 (segment (start 200.96 83.5) (end 200.44 83.5) (width 2) (layer "B.Cu") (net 1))
 (segment (start 215.8 73.5) (end 220.5 73.5) (width 2) (layer "B.Cu") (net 1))
 (segment (start 169.46 76.62) (end 164.5 71.66) (width 2) (layer "F.Cu") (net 2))
 (segment (start 169.46 82.54) (end 169.46 76.62) (width 2) (layer "F.Cu") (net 2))
 (segment (start 169.46 82.54) (end 169.5 82.58) (width 2) (layer "F.Cu") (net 2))
 (via (at 169.46 82.54) (size 2.5) (drill 0.5) (layers "F.Cu" "B.Cu") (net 2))
 (segment (start 204 86.5) (end 203.41 85.91) (width 2) (layer "B.Cu") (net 2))
 (segment (start 204 86.5) (end 208.75 86.5) (width 2) (layer "B.Cu") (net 2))
 (segment (start 169.46 82.54) (end 171 84.08) (width 2) (layer "B.Cu") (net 2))
 (segment (start 208.75 83.25) (end 208.75 86.5) (width 2) (layer "B.Cu") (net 2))
 (segment (start 172.5 91) (end 197.5 91) (width 2) (layer "B.Cu") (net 2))
 (segment (start 203.41 85.91) (end 200.31 85.91) (width 2) (layer "B.Cu") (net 2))
 (segment (start 171 84.08) (end 171 89.5) (width 2) (layer "B.Cu") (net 2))
 (segment (start 207.5 82) (end 208.75 83.25) (width 2) (layer "B.Cu") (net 2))
 (segment (start 200.4 86) (end 200.31 85.91) (width 1.5) (layer "B.Cu") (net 2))
 (segment (start 207.5 75) (end 207.5 82) (width 2) (layer "B.Cu") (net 2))
 (segment (start 200.31 88.19) (end 200.31 85.91) (width 2) (layer "B.Cu") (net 2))
 (segment (start 171 89.5) (end 172.5 91) (width 2) (layer "B.Cu") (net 2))
 (segment (start 197.5 91) (end 200.31 88.19) (width 2) (layer "B.Cu") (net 2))
 (segment (start 183 46) (end 181.5 47.5) (width 2) (layer "F.Cu") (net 25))
 (segment (start 171.5 62.5) (end 167.42 66.58) (width 2) (layer "F.Cu") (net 25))
 (segment (start 171.5 52.5) (end 171.5 62.5) (width 2) (layer "F.Cu") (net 25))
 (segment (start 197 46) (end 183 46) (width 2) (layer "F.Cu") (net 25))
 (segment (start 176.5 47.5) (end 171.5 52.5) (width 2) (layer "F.Cu") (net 25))
 (segment (start 167.42 66.58) (end 164.5 66.58) (width 2) (layer "F.Cu") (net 25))
 (segment (start 202 48) (end 199 48) (width 2) (layer "F.Cu") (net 25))
 (segment (start 181.5 47.5) (end 176.5 47.5) (width 2) (layer "F.Cu") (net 25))
 (segment (start 199 48) (end 197 46) (width 2) (layer "F.Cu") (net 25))
 (via (at 202 48) (size 2) (drill 0.5) (layers "F.Cu" "B.Cu") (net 25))
 (segment (start 202.5 48.5) (end 202.5 50.2) (width 2) (layer "B.Cu") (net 25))
 (segment (start 202 48) (end 202.5 48.5) (width 2) (layer "B.Cu") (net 25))
 (segment (start 202.5 50.2) (end 202.5 50.7) (width 1.4) (layer "B.Cu") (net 25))
 (segment (start 202.5 50.7) (end 200.31 52.89) (width 1.4) (layer "B.Cu") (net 25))
 (segment (start 200.95 63.05) (end 200.31 63.05) (width 1.4) (layer "B.Cu") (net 4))
 (segment (start 206.46 57.54) (end 200.95 63.05) (width 1.4) (layer "B.Cu") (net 4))
 (segment (start 206.23 67) (end 206.5 67.27) (width 1.5) (layer "B.Cu") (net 4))
 (segment (start 202 67) (end 206.23 67) (width 1.5) (layer "B.Cu") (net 4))
 (segment (start 200.87 68.13) (end 202 67) (width 1.5) (layer "B.Cu") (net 4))
 (segment (start 200.31 68.13) (end 200.87 68.13) (width 1.5) (layer "B.Cu") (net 4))
 (segment (start 206.46 53) (end 206.46 57.54) (width 1.4) (layer "B.Cu") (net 4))
 (segment (start 179 44.5) (end 176 44.5) (width 2) (layer "F.Cu") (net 22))
 (segment (start 205 46) (end 204 45) (width 2) (layer "F.Cu") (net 22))
 (segment (start 198.5 43) (end 180.5 43) (width 2) (layer "F.Cu") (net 22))
 (segment (start 204 45) (end 200.5 45) (width 2) (layer "F.Cu") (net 22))
 (segment (start 165.96 64.04) (end 164.5 64.04) (width 2) (layer "F.Cu") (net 22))
 (segment (start 176 44.5) (end 168 52.5) (width 2) (layer "F.Cu") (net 22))
 (segment (start 168 62) (end 165.96 64.04) (width 2) (layer "F.Cu") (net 22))
 (segment (start 200.5 45) (end 198.5 43) (width 2) (layer "F.Cu") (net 22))
 (segment (start 180.5 43) (end 179 44.5) (width 2) (layer "F.Cu") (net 22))
 (segment (start 168 52.5) (end 168 62) (width 2) (layer "F.Cu") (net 22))
 (via (at 205 46) (size 2) (drill 0.5) (layers "F.Cu" "B.Cu") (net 22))
 (segment (start 205 50.5) (end 204.5 51) (width 1.3) (layer "B.Cu") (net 22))
 (segment (start 204.5 51) (end 204.5 56.5) (width 1.3) (layer "B.Cu") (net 22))
 (segment (start 204.5 56.5) (end 202.68 58.32) (width 1.3) (layer "B.Cu") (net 22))
 (segment (start 202.68 58.32) (end 202.5 58.32) (width 1.3) (layer "B.Cu") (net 22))
 (segment (start 205 46) (end 205 50.5) (width 2) (layer "B.Cu") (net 22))
 (segment (start 202.5 58.32) (end 200.31 60.51) (width 1.3) (layer "B.Cu") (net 22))
 (segment (start 200.31 60.44) (end 200.31 60.51) (width 0.2) (layer "B.Cu") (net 22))
 (segment (start 209.5 57) (end 212.6 57) (width 2) (layer "B.Cu") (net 3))
 (segment (start 215.5 63) (end 213.3 63) (width 2) (layer "B.Cu") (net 3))
 (segment (start 213.3 57.7) (end 213.3 63) (width 2) (layer "B.Cu") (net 3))
 (segment (start 216.5 67.5) (end 216.5 64) (width 2) (layer "B.Cu") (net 3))
 (segment (start 212.75 72.75) (end 212.75 80.5) (width 2) (layer "B.Cu") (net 3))
 (segment (start 215.5 68.5) (end 216.5 67.5) (width 2) (layer "B.Cu") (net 3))
 (segment (start 209 53) (end 209 56.5) (width 2) (layer "B.Cu") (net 3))
 (segment (start 210.04 74.96) (end 215.5 69.5) (width 2) (layer "B.Cu") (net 3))
 (segment (start 210.04 75) (end 210.04 74.96) (width 1) (layer "B.Cu") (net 3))
 (segment (start 209 56.5) (end 209.5 57) (width 2) (layer "B.Cu") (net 3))
 (segment (start 212.6 57) (end 213.3 57.7) (width 2) (layer "B.Cu") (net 3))
 (segment (start 216.5 64) (end 215.5 63) (width 2) (layer "B.Cu") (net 3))
 (segment (start 209.5 59.19) (end 206.5 62.19) (width 2) (layer "B.Cu") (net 3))
 (segment (start 209.5 57) (end 209.5 59.19) (width 2) (layer "B.Cu") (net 3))
 (segment (start 215.5 69.5) (end 215.5 68.5) (width 2) (layer "B.Cu") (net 3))
 (segment (start 200.31 65.59) (end 200.82 65.59) (width 1.4) (layer "B.Cu") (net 5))
 (segment (start 206.23 65) (end 206.5 64.73) (width 1.4) (layer "B.Cu") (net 5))
 (segment (start 200.82 65.59) (end 201.41 65) (width 1.4) (layer "B.Cu") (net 5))
 (segment (start 201.41 65) (end 206.23 65) (width 1.4) (layer "B.Cu") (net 5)))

